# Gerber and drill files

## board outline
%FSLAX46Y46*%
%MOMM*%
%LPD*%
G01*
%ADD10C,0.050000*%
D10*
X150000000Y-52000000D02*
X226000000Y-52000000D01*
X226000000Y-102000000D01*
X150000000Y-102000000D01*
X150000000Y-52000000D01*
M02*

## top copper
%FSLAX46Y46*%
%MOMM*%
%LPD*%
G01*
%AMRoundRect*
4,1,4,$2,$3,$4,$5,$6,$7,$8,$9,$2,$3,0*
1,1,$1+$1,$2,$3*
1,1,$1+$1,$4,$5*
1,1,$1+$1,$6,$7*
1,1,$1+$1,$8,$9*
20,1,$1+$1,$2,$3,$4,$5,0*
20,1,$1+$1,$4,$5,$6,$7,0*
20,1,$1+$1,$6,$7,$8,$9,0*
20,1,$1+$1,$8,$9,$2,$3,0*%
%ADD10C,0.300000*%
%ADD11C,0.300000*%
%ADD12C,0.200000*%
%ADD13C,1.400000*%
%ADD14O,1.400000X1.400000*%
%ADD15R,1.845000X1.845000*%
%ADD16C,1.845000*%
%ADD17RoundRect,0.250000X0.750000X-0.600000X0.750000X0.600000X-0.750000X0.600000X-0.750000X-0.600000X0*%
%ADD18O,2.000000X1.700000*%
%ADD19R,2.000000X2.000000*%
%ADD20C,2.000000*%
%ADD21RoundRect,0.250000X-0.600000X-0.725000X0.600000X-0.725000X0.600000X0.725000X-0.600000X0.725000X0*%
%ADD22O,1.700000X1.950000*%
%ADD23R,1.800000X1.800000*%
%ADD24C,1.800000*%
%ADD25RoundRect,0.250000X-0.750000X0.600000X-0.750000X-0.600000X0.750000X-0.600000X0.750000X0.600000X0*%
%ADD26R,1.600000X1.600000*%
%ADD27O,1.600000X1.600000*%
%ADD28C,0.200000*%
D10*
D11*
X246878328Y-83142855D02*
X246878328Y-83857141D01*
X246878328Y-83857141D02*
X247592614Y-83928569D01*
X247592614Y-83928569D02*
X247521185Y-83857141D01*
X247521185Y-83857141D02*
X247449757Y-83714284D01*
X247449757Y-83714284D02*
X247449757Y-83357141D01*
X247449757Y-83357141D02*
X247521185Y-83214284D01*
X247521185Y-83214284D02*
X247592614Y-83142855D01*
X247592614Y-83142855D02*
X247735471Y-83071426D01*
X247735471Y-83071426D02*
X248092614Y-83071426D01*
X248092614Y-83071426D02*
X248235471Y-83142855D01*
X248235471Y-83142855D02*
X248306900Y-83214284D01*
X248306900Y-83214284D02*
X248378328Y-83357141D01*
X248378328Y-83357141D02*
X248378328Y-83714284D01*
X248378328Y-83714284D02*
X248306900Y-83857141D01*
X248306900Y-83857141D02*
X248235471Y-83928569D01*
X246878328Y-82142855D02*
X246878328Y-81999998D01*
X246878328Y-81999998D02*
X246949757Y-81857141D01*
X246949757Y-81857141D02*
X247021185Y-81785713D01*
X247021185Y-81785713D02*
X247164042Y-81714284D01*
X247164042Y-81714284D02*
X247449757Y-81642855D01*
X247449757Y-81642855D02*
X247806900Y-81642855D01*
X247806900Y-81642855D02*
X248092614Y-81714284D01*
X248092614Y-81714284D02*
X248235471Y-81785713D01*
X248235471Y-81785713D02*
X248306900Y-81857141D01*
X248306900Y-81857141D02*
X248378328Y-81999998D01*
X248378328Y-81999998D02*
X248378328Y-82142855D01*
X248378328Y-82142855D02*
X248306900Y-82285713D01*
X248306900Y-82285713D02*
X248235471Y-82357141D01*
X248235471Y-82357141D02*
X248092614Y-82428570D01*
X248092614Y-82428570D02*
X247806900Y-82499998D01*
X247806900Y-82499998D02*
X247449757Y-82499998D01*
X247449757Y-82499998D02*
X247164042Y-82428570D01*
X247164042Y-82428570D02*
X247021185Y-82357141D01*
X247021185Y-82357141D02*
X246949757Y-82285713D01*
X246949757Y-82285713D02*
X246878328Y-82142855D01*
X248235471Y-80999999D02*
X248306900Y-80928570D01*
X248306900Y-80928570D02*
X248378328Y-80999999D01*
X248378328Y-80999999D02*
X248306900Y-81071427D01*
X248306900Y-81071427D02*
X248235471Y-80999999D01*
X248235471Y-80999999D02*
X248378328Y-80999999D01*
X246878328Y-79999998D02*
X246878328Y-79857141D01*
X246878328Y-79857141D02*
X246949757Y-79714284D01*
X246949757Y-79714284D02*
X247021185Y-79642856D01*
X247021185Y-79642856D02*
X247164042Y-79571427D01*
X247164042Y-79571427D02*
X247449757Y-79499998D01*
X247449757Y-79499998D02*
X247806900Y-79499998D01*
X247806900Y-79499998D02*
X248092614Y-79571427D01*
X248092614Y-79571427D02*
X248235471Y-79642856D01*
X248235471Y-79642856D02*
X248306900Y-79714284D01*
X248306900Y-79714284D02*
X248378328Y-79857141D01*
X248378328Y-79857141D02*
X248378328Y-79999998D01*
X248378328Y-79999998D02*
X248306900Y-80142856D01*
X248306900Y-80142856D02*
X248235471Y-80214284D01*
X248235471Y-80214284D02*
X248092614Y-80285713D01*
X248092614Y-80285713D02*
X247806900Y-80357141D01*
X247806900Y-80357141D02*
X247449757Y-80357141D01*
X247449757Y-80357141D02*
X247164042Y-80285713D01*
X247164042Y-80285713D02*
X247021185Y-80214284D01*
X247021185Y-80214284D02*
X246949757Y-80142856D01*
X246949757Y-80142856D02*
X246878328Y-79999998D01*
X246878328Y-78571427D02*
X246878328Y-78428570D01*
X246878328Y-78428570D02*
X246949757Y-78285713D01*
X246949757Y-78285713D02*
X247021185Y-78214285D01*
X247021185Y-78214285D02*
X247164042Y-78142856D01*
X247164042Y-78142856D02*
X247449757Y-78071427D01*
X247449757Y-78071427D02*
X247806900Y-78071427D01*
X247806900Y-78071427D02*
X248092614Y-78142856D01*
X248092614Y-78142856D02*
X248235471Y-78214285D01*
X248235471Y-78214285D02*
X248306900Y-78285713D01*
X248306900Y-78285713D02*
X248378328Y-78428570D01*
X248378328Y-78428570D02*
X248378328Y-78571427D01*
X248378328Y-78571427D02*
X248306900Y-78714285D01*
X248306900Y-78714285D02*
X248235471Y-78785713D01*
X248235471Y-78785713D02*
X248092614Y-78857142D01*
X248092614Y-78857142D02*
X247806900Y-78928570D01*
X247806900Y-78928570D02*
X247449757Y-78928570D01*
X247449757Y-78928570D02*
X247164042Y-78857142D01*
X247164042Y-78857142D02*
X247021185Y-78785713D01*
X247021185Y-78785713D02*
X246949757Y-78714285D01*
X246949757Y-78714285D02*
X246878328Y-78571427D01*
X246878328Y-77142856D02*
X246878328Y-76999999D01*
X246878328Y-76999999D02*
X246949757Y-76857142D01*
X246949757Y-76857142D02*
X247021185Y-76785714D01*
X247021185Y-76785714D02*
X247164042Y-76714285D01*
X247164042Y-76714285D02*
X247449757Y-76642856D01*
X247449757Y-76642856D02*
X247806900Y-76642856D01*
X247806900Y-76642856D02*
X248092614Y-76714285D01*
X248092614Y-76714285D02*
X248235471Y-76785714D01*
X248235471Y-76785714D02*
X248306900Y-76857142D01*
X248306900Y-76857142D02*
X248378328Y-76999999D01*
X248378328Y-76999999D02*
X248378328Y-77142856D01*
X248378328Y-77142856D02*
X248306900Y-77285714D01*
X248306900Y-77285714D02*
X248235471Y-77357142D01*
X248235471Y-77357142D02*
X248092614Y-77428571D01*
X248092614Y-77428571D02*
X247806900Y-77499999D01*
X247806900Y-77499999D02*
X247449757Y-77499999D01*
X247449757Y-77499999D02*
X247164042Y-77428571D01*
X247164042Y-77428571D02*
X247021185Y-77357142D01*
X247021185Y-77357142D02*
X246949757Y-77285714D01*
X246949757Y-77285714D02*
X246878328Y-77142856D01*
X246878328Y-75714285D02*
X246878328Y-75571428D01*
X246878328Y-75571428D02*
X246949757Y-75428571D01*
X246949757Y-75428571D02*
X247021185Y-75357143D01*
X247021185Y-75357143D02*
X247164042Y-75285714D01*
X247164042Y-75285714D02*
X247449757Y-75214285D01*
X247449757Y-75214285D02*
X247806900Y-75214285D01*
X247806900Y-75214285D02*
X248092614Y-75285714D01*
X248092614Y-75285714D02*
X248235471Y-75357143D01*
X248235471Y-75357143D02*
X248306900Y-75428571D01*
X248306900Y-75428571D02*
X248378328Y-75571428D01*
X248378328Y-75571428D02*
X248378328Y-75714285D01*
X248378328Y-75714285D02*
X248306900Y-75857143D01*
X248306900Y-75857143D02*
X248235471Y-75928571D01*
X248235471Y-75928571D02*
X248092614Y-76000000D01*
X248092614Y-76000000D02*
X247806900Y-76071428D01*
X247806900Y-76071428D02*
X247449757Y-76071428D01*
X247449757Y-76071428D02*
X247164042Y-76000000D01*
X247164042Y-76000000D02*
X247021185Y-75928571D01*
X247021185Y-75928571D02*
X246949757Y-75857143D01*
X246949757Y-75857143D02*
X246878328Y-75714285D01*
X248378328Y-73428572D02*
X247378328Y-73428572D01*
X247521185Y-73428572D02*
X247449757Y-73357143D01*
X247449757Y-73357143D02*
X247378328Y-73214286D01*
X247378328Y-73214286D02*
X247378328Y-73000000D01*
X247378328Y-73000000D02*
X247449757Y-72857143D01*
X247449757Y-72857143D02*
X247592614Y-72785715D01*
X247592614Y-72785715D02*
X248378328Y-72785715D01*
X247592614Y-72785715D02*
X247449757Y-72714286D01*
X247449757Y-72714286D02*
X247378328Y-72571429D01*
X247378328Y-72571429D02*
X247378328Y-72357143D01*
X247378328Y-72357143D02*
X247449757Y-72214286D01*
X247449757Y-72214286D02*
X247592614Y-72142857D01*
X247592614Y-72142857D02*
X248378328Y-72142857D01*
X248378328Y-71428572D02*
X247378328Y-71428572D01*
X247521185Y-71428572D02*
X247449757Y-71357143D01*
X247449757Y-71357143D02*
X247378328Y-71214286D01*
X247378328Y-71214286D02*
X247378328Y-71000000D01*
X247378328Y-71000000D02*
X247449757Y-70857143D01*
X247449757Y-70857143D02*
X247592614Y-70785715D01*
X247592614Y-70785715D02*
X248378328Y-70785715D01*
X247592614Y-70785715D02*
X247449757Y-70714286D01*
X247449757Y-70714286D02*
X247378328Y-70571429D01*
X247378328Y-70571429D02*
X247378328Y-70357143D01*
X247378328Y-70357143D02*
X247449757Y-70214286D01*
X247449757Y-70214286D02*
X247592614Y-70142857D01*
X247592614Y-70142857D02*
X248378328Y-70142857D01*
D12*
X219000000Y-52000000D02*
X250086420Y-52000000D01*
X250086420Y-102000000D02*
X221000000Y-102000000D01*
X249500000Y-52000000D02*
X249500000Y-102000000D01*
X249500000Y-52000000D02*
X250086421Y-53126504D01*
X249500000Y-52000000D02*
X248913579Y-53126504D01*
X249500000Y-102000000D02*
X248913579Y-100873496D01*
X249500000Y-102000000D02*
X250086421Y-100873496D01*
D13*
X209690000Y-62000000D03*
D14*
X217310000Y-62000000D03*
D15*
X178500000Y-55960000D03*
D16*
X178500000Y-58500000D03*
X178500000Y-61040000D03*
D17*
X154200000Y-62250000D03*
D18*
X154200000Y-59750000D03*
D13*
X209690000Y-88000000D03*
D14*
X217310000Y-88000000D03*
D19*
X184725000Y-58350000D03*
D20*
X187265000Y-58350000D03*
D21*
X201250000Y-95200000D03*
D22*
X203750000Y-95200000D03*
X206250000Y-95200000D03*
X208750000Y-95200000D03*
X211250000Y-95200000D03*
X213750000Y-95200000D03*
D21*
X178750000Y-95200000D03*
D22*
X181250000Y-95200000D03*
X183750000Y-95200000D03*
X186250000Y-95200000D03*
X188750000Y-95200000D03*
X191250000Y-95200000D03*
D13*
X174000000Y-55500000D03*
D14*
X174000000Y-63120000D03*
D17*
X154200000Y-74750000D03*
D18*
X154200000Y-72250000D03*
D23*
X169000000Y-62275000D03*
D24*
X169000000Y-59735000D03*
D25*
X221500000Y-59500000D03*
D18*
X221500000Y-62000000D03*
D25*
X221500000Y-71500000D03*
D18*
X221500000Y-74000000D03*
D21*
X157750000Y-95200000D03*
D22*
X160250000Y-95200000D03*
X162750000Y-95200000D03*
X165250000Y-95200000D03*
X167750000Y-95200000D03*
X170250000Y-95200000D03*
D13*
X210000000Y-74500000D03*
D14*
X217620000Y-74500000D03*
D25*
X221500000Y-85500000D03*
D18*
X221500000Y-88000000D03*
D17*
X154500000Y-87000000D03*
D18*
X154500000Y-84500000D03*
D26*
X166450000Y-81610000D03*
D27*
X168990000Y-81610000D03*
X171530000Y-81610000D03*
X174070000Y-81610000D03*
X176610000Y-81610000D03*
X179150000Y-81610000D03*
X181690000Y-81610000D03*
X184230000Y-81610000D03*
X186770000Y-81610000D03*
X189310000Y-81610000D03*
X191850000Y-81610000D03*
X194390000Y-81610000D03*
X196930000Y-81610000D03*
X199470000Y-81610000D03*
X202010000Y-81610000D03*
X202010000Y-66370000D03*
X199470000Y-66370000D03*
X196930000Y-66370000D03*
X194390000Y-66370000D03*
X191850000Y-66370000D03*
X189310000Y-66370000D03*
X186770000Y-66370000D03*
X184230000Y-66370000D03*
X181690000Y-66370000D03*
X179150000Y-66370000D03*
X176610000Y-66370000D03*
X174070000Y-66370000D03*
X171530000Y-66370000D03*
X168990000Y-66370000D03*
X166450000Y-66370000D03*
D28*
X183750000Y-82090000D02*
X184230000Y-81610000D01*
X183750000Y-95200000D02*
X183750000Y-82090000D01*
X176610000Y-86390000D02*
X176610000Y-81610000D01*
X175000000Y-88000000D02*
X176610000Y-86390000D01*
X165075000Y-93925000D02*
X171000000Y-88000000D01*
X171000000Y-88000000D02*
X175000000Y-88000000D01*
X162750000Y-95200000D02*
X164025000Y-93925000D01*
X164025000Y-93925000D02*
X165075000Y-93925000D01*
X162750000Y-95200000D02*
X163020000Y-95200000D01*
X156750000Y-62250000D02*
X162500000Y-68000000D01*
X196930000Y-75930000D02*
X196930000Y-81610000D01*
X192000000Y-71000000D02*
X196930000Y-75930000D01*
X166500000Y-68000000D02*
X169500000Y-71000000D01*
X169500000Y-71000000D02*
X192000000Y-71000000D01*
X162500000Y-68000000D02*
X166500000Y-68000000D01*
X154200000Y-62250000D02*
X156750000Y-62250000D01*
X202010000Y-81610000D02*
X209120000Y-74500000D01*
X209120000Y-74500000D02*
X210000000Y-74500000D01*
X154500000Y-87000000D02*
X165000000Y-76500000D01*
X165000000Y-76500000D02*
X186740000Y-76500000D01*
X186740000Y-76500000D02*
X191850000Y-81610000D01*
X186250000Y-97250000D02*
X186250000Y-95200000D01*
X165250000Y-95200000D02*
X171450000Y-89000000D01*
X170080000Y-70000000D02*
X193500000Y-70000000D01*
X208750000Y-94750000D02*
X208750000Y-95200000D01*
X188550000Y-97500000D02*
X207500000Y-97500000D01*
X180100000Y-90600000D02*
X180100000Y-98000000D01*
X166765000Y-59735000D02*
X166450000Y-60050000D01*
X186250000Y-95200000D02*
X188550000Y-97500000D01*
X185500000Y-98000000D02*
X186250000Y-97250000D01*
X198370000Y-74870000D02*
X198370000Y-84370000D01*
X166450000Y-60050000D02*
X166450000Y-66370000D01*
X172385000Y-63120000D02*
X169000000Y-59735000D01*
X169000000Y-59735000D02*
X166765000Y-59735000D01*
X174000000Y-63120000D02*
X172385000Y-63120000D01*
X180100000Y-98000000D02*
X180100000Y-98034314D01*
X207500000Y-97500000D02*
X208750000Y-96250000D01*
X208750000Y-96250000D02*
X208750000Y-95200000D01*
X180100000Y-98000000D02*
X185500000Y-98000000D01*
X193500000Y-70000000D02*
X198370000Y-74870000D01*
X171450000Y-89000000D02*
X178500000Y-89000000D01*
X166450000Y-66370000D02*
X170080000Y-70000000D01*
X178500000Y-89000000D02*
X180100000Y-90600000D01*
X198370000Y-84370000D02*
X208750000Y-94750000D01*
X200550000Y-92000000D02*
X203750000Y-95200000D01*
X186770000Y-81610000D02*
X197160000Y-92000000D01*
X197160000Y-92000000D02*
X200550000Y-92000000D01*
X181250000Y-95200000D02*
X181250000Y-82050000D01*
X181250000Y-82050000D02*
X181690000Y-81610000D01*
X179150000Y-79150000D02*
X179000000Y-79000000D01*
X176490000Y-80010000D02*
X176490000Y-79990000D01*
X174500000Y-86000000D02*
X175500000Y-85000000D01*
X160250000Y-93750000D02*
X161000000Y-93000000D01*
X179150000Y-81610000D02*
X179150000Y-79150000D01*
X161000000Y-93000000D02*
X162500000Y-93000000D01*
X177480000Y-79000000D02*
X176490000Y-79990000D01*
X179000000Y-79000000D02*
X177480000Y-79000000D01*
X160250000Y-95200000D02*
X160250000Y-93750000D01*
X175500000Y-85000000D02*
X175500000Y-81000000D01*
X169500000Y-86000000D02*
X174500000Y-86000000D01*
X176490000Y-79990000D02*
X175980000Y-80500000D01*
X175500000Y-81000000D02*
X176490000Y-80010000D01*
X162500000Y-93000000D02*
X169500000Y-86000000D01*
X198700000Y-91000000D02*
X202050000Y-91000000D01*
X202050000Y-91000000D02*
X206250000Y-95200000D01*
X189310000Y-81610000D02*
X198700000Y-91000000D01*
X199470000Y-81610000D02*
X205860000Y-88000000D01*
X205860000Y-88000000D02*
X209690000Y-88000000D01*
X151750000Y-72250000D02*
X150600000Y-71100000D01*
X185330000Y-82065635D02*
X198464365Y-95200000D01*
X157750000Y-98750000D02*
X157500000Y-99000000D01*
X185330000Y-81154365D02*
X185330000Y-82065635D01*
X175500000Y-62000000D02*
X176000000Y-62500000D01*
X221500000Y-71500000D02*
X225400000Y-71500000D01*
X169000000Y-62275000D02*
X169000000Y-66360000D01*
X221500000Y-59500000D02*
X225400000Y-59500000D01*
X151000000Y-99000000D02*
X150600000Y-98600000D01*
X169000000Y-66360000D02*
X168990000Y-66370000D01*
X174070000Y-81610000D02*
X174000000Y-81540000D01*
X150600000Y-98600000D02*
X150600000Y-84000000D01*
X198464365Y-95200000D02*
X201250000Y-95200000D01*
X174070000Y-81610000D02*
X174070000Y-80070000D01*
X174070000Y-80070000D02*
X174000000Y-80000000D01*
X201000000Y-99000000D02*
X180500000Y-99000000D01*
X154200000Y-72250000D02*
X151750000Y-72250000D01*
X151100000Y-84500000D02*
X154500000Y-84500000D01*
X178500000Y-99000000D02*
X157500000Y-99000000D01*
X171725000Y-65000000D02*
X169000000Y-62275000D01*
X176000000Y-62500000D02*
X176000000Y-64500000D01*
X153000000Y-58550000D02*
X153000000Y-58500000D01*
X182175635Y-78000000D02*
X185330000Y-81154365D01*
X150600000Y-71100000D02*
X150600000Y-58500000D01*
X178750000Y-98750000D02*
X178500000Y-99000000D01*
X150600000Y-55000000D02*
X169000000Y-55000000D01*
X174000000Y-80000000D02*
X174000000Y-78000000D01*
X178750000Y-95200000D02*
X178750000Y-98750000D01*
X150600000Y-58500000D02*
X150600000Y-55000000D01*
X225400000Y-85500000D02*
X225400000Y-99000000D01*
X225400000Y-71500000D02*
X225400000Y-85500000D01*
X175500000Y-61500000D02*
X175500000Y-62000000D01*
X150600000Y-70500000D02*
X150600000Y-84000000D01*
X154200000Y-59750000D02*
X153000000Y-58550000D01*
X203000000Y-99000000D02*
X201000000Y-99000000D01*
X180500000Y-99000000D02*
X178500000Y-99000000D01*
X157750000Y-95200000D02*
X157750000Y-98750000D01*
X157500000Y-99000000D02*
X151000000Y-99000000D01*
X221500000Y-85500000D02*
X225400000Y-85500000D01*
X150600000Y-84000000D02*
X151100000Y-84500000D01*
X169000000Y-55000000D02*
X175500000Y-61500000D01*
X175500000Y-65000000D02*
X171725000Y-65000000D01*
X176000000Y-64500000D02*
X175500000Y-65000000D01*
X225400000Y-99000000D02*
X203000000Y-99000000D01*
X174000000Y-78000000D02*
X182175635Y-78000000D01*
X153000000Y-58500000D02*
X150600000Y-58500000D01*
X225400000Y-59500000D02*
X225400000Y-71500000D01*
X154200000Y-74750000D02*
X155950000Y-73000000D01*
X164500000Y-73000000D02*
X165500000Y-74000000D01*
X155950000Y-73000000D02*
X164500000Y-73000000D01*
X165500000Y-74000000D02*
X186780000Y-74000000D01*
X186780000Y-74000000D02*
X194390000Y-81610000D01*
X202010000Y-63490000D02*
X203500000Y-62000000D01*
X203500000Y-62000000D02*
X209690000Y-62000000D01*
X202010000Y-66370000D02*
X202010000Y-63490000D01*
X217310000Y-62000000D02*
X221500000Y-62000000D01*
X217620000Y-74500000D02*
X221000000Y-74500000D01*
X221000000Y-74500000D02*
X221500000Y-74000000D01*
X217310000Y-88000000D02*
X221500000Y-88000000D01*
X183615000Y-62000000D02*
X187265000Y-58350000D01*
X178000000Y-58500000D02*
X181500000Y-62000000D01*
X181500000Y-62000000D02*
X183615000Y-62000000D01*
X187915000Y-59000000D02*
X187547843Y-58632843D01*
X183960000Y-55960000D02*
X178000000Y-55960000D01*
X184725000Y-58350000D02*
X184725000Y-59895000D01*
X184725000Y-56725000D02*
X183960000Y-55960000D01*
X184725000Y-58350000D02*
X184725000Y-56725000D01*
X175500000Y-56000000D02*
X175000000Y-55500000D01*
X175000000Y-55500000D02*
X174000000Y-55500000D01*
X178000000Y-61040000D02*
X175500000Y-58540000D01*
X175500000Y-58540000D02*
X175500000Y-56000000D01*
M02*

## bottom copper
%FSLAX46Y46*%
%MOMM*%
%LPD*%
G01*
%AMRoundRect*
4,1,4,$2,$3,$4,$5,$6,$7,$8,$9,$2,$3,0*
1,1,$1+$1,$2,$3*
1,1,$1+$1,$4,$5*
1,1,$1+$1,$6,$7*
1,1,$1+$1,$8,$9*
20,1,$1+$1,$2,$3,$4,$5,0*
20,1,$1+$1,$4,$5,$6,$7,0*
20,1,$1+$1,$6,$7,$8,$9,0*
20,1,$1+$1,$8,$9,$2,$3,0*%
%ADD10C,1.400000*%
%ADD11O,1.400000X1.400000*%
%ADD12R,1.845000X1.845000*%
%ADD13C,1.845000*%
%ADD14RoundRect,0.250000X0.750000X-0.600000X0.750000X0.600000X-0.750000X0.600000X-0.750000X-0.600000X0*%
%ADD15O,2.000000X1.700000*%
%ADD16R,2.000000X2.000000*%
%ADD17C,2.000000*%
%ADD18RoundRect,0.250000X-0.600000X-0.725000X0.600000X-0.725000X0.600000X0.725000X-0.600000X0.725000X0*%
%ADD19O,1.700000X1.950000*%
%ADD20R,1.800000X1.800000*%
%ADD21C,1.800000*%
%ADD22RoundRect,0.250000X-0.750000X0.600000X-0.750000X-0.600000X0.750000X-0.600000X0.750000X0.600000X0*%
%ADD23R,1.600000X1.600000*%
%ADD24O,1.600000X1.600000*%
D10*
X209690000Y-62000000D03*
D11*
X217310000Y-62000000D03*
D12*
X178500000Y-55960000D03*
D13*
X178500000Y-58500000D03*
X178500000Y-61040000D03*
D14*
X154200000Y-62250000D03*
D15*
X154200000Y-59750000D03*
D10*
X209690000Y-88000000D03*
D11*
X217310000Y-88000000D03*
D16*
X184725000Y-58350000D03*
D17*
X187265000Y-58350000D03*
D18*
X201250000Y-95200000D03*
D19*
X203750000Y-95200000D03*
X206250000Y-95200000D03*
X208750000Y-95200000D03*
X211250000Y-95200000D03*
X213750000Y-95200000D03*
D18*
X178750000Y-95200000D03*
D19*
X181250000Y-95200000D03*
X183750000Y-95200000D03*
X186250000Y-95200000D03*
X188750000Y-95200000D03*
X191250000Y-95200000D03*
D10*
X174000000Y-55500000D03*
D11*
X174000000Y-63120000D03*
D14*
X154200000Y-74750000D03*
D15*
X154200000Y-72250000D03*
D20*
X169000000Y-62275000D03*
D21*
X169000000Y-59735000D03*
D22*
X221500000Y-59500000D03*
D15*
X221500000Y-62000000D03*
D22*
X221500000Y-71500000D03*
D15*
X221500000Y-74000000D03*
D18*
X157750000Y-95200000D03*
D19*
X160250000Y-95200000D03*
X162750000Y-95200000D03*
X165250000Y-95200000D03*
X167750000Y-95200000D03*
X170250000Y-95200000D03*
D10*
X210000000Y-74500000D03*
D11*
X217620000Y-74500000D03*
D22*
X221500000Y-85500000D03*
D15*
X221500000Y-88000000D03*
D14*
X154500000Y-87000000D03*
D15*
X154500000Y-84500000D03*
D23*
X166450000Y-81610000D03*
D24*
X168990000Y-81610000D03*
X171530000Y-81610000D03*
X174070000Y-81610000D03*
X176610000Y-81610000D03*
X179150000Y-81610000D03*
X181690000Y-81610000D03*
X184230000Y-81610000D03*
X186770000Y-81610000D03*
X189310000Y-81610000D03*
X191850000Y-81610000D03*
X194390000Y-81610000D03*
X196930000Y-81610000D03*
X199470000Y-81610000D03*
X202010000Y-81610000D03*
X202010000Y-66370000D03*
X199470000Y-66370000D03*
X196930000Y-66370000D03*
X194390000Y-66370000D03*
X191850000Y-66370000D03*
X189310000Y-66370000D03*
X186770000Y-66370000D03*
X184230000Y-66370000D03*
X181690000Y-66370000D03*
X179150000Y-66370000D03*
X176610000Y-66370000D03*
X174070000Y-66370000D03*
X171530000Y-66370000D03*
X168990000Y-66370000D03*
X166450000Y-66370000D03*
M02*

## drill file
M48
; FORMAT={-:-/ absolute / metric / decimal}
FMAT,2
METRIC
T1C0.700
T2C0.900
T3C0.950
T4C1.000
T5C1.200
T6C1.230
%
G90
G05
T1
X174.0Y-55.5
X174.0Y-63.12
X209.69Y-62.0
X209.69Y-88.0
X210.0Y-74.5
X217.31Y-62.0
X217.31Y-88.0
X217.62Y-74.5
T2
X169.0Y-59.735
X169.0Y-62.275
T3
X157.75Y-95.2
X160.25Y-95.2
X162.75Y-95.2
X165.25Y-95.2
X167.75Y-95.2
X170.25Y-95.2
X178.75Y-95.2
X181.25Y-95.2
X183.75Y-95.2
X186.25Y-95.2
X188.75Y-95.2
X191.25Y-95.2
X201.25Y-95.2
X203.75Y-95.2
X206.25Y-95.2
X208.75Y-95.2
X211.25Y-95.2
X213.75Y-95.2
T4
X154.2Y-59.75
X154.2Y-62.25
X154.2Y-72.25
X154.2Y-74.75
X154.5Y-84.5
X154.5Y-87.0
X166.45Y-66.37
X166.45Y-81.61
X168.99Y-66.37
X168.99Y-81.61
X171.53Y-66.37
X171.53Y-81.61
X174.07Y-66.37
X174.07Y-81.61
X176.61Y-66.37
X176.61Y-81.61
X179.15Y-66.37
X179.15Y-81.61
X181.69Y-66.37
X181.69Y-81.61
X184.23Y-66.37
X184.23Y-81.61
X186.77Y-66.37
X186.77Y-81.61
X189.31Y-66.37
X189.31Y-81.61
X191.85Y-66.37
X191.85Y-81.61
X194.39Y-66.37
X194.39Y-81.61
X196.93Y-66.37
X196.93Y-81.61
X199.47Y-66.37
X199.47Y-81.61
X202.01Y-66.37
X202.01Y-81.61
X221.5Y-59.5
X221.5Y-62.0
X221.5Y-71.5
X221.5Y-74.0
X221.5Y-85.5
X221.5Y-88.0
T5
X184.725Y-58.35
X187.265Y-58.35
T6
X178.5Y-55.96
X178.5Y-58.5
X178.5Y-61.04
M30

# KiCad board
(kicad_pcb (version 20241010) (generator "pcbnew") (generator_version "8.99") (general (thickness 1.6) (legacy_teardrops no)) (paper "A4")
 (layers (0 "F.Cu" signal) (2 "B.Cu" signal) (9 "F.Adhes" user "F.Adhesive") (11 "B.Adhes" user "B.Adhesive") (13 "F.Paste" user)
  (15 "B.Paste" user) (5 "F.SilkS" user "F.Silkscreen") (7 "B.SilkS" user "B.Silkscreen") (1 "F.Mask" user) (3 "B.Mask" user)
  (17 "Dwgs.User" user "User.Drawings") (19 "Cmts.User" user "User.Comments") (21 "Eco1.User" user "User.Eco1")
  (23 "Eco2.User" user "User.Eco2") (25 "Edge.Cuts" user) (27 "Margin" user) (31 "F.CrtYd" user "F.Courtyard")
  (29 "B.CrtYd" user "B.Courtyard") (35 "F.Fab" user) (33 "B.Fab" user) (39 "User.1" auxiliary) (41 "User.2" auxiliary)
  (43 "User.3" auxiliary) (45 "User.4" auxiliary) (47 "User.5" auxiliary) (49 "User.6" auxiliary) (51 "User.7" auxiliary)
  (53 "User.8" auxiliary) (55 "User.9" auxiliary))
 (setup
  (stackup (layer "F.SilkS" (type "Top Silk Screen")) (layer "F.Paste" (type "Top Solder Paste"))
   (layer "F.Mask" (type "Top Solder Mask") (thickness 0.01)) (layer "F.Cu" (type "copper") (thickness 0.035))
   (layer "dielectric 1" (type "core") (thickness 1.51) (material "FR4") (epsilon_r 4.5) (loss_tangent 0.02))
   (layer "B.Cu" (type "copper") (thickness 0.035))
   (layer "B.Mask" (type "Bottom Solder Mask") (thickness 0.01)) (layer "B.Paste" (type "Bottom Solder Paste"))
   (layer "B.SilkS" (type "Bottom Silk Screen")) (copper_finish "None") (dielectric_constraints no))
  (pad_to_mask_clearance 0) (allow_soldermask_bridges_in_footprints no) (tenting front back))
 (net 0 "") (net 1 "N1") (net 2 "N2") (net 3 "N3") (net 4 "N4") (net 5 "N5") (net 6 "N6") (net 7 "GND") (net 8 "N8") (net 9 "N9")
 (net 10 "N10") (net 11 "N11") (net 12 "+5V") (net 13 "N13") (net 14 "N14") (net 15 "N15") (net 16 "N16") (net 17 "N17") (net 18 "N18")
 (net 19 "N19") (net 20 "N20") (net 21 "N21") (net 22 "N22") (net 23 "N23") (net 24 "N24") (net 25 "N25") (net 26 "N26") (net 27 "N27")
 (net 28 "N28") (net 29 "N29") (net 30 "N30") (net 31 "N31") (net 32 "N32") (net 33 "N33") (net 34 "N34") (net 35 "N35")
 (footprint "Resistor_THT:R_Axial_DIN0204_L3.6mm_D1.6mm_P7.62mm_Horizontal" (layer "F.Cu") (at 209.69 62)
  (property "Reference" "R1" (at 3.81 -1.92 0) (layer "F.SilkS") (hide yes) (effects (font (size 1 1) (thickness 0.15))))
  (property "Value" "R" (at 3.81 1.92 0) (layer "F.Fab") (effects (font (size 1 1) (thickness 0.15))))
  (pad "1" thru_hole circle (at 0 0) (size 1.4 1.4) (drill 0.7) (layers "*.Cu" "*.Mask") (remove_unused_layers no) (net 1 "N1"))
  (pad "2" thru_hole oval (at 7.62 0) (size 1.4 1.4) (drill 0.7) (layers "*.Cu" "*.Mask") (remove_unused_layers no) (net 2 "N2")))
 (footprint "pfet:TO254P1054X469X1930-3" (layer "F.Cu") (at 179.3105 58.5 -90)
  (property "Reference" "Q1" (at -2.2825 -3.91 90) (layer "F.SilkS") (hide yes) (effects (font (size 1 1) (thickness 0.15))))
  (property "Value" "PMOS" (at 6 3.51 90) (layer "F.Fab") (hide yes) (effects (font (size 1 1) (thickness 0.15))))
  (pad "1" thru_hole rect (at -2.54 0.8105 270) (size 1.845 1.845) (drill 1.23) (layers "*.Cu" "*.Mask") (remove_unused_layers no)
   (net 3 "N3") (solder_mask_margin 0.102))
  (pad "2" thru_hole circle (at 0 0.8105 270) (size 1.845 1.845) (drill 1.23) (layers "*.Cu" "*.Mask") (remove_unused_layers no)
   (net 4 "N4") (solder_mask_margin 0.102))
  (pad "3" thru_hole circle (at 2.54 0.8105 270) (size 1.845 1.845) (drill 1.23) (layers "*.Cu" "*.Mask") (remove_unused_layers no)
   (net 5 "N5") (solder_mask_margin 0.102)))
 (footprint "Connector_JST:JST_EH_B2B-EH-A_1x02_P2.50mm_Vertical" (layer "F.Cu") (at 154.2 62.25 90)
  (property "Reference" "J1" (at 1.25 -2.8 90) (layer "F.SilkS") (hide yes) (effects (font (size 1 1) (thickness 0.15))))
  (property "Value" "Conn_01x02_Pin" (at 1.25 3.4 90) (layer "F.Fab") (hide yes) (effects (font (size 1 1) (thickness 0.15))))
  (pad "1" thru_hole roundrect (at 0 0 90) (size 1.7 2) (drill 1) (layers "*.Cu" "*.Mask") (remove_unused_layers no)
   (roundrect_rratio 0.147059) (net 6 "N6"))
  (pad "2" thru_hole oval (at 2.5 0 90) (size 1.7 2) (drill 1) (layers "*.Cu" "*.Mask") (remove_unused_layers no) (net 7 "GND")))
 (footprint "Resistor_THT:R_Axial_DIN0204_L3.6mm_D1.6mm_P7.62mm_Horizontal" (layer "F.Cu") (at 209.69 88)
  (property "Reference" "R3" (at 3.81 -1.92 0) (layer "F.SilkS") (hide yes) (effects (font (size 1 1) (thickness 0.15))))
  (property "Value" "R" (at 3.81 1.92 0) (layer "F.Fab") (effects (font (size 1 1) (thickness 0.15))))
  (pad "1" thru_hole circle (at 0 0) (size 1.4 1.4) (drill 0.7) (layers "*.Cu" "*.Mask") (remove_unused_layers no) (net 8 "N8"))
  (pad "2" thru_hole oval (at 7.62 0) (size 1.4 1.4) (drill 0.7) (layers "*.Cu" "*.Mask") (remove_unused_layers no) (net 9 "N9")))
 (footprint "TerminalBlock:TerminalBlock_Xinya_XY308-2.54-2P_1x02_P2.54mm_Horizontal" (layer "F.Cu") (at 184.725 58.35)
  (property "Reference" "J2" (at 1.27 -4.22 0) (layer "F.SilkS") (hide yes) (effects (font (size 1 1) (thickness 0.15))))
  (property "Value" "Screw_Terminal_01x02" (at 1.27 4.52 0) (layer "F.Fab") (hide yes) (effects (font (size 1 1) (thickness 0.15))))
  (pad "1" thru_hole rect (at 0 0) (size 2 2) (drill 1.2) (layers "*.Cu" "*.Mask") (remove_unused_layers no) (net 3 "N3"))
  (pad "2" thru_hole circle (at 2.54 0) (size 2 2) (drill 1.2) (layers "*.Cu" "*.Mask") (remove_unused_layers no) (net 4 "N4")))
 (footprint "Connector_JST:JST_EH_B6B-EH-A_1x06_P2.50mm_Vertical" (layer "F.Cu") (at 201.25 95.2)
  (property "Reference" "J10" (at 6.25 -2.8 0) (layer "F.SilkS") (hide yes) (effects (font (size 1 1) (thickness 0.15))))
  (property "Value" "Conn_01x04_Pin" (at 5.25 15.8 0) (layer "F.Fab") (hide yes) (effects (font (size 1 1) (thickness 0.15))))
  (pad "1" thru_hole roundrect (at 0 0) (size 1.7 1.95) (drill 0.95) (layers "*.Cu" "*.Mask") (remove_unused_layers no)
   (roundrect_rratio 0.147059) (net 7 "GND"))
  (pad "2" thru_hole oval (at 2.5 0) (size 1.7 1.95) (drill 0.95) (layers "*.Cu" "*.Mask") (remove_unused_layers no) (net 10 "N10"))
  (pad "3" thru_hole oval (at 5 0) (size 1.7 1.95) (drill 0.95) (layers "*.Cu" "*.Mask") (remove_unused_layers no) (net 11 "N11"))
  (pad "4" thru_hole oval (at 7.5 0) (size 1.7 1.95) (drill 0.95) (layers "*.Cu" "*.Mask") (remove_unused_layers no) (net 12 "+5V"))
  (pad "5" thru_hole oval (at 10 0) (size 1.7 1.95) (drill 0.95) (layers "*.Cu" "*.Mask") (remove_unused_layers no))
  (pad "6" thru_hole oval (at 12.5 0) (size 1.7 1.95) (drill 0.95) (layers "*.Cu" "*.Mask") (remove_unused_layers no)))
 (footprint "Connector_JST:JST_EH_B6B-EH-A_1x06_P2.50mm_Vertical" (layer "F.Cu") (at 178.75 95.2)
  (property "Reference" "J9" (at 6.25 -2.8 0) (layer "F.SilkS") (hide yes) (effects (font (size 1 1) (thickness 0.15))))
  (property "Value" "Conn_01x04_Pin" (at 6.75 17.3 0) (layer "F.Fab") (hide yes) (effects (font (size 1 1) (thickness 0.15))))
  (pad "1" thru_hole roundrect (at 0 0) (size 1.7 1.95) (drill 0.95) (layers "*.Cu" "*.Mask") (remove_unused_layers no)
   (roundrect_rratio 0.147059) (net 7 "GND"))
  (pad "2" thru_hole oval (at 2.5 0) (size 1.7 1.95) (drill 0.95) (layers "*.Cu" "*.Mask") (remove_unused_layers no) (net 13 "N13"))
  (pad "3" thru_hole oval (at 5 0) (size 1.7 1.95) (drill 0.95) (layers "*.Cu" "*.Mask") (remove_unused_layers no) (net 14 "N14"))
  (pad "4" thru_hole oval (at 7.5 0) (size 1.7 1.95) (drill 0.95) (layers "*.Cu" "*.Mask") (remove_unused_layers no) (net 12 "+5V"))
  (pad "5" thru_hole oval (at 10 0) (size 1.7 1.95) (drill 0.95) (layers "*.Cu" "*.Mask") (remove_unused_layers no))
  (pad "6" thru_hole oval (at 12.5 0) (size 1.7 1.95) (drill 0.95) (layers "*.Cu" "*.Mask") (remove_unused_layers no)))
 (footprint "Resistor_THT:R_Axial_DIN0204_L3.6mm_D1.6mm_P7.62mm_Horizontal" (layer "F.Cu") (at 174 55.5 -90)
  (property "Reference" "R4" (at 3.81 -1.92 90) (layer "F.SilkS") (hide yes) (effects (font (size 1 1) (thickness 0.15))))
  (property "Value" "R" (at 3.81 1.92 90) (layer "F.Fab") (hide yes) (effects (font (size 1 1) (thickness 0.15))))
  (pad "1" thru_hole circle (at 0 0 270) (size 1.4 1.4) (drill 0.7) (layers "*.Cu" "*.Mask") (remove_unused_layers no) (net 5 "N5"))
  (pad "2" thru_hole oval (at 7.62 0 270) (size 1.4 1.4) (drill 0.7) (layers "*.Cu" "*.Mask") (remove_unused_layers no) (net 12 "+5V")))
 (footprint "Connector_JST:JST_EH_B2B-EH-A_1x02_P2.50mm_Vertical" (layer "F.Cu") (at 154.2 74.75 90)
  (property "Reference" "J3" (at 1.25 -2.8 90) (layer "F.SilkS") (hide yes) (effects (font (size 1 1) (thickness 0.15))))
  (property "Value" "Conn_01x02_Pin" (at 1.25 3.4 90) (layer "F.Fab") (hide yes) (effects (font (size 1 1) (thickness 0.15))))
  (pad "1" thru_hole roundrect (at 0 0 90) (size 1.7 2) (drill 1) (layers "*.Cu" "*.Mask") (remove_unused_layers no)
   (roundrect_rratio 0.147059) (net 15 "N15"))
  (pad "2" thru_hole oval (at 2.5 0 90) (size 1.7 2) (drill 1) (layers "*.Cu" "*.Mask") (remove_unused_layers no) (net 7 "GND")))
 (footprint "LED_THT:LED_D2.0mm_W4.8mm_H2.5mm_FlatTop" (layer "F.Cu") (at 169 62.275 90)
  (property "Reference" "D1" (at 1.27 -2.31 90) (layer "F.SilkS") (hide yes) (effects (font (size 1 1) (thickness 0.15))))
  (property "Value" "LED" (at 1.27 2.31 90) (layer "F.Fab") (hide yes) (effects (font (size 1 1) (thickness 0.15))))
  (pad "1" thru_hole rect (at 0 0 90) (size 1.8 1.8) (drill 0.9) (layers "*.Cu" "*.Mask") (remove_unused_layers no) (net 7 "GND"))
  (pad "2" thru_hole circle (at 2.54 0 90) (size 1.8 1.8) (drill 0.9) (layers "*.Cu" "*.Mask") (remove_unused_layers no) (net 12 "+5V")))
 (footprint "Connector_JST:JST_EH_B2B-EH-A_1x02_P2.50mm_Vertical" (layer "F.Cu") (at 221.5 59.5 -90)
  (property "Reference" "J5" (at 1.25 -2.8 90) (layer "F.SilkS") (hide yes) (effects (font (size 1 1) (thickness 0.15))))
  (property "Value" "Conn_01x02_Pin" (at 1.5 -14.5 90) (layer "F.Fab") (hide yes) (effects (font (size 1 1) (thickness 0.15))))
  (pad "1" thru_hole roundrect (at 0 0 270) (size 1.7 2) (drill 1) (layers "*.Cu" "*.Mask") (remove_unused_layers no)
   (roundrect_rratio 0.147059) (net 7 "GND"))
  (pad "2" thru_hole oval (at 2.5 0 270) (size 1.7 2) (drill 1) (layers "*.Cu" "*.Mask") (remove_unused_layers no) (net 2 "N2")))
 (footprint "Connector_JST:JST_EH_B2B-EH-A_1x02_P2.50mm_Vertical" (layer "F.Cu") (at 221.5 71.5 -90)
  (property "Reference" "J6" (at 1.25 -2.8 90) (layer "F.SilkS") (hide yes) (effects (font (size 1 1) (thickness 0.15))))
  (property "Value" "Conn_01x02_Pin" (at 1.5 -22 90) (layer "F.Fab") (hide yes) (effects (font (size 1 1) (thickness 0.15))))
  (pad "1" thru_hole roundrect (at 0 0 270) (size 1.7 2) (drill 1) (layers "*.Cu" "*.Mask") (remove_unused_layers no)
   (roundrect_rratio 0.147059) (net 7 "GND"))
  (pad "2" thru_hole oval (at 2.5 0 270) (size 1.7 2) (drill 1) (layers "*.Cu" "*.Mask") (remove_unused_layers no) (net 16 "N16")))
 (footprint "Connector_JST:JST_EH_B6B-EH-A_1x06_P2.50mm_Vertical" (layer "F.Cu") (at 157.75 95.2)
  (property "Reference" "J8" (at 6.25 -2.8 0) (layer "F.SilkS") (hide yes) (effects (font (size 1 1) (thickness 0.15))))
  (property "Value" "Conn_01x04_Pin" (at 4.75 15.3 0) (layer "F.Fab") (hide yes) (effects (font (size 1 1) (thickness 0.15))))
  (pad "1" thru_hole roundrect (at 0 0) (size 1.7 1.95) (drill 0.95) (layers "*.Cu" "*.Mask") (remove_unused_layers no)
   (roundrect_rratio 0.147059) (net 7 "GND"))
  (pad "2" thru_hole oval (at 2.5 0) (size 1.7 1.95) (drill 0.95) (layers "*.Cu" "*.Mask") (remove_unused_layers no) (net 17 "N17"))
  (pad "3" thru_hole oval (at 5 0) (size 1.7 1.95) (drill 0.95) (layers "*.Cu" "*.Mask") (remove_unused_layers no) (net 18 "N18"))
  (pad "4" thru_hole oval (at 7.5 0) (size 1.7 1.95) (drill 0.95) (layers "*.Cu" "*.Mask") (remove_unused_layers no) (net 12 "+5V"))
  (pad "5" thru_hole oval (at 10 0) (size 1.7 1.95) (drill 0.95) (layers "*.Cu" "*.Mask") (remove_unused_layers no))
  (pad "6" thru_hole oval (at 12.5 0) (size 1.7 1.95) (drill 0.95) (layers "*.Cu" "*.Mask") (remove_unused_layers no)))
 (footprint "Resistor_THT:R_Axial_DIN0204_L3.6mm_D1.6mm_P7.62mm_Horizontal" (layer "F.Cu") (at 210 74.5)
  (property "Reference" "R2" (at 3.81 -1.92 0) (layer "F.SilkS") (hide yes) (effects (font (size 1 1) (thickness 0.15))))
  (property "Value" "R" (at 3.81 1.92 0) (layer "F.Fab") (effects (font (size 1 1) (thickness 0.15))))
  (pad "1" thru_hole circle (at 0 0) (size 1.4 1.4) (drill 0.7) (layers "*.Cu" "*.Mask") (remove_unused_layers no) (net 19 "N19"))
  (pad "2" thru_hole oval (at 7.62 0) (size 1.4 1.4) (drill 0.7) (layers "*.Cu" "*.Mask") (remove_unused_layers no) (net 16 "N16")))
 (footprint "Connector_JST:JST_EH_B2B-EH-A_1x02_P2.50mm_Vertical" (layer "F.Cu") (at 221.5 85.5 -90)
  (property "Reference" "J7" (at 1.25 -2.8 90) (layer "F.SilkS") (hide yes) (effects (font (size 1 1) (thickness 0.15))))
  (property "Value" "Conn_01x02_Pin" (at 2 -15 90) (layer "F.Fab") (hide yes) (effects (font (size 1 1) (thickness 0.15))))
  (pad "1" thru_hole roundrect (at 0 0 270) (size 1.7 2) (drill 1) (layers "*.Cu" "*.Mask") (remove_unused_layers no)
   (roundrect_rratio 0.147059) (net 7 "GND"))
  (pad "2" thru_hole oval (at 2.5 0 270) (size 1.7 2) (drill 1) (layers "*.Cu" "*.Mask") (remove_unused_layers no) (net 9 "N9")))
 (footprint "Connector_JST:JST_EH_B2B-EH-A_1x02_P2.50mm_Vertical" (layer "F.Cu") (at 154.5 87 90)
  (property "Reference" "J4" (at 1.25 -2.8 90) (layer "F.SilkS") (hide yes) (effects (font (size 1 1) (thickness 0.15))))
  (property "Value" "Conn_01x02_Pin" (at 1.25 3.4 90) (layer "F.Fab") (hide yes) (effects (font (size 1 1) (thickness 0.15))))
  (pad "1" thru_hole roundrect (at 0 0 90) (size 1.7 2) (drill 1) (layers "*.Cu" "*.Mask") (remove_unused_layers no)
   (roundrect_rratio 0.147059) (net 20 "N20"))
  (pad "2" thru_hole oval (at 2.5 0 90) (size 1.7 2) (drill 1) (layers "*.Cu" "*.Mask") (remove_unused_layers no) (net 7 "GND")))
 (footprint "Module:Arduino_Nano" (layer "F.Cu") (at 166.45 81.61 90)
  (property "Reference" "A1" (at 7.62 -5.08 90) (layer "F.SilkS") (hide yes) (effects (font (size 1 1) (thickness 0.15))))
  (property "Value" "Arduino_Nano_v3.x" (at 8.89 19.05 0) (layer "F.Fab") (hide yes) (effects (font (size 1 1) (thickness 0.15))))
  (pad "1" thru_hole rect (at 0 0 90) (size 1.6 1.6) (drill 1) (layers "*.Cu" "*.Mask") (remove_unused_layers no) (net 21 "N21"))
  (pad "2" thru_hole oval (at 0 2.54 90) (size 1.6 1.6) (drill 1) (layers "*.Cu" "*.Mask") (remove_unused_layers no) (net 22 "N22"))
  (pad "3" thru_hole oval (at 0 5.08 90) (size 1.6 1.6) (drill 1) (layers "*.Cu" "*.Mask") (remove_unused_layers no) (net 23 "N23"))
  (pad "4" thru_hole oval (at 0 7.62 90) (size 1.6 1.6) (drill 1) (layers "*.Cu" "*.Mask") (remove_unused_layers no) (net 7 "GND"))
  (pad "5" thru_hole oval (at 0 10.16 90) (size 1.6 1.6) (drill 1) (layers "*.Cu" "*.Mask") (remove_unused_layers no) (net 18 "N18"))
  (pad "6" thru_hole oval (at 0 12.7 90) (size 1.6 1.6) (drill 1) (layers "*.Cu" "*.Mask") (remove_unused_layers no) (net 17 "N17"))
  (pad "7" thru_hole oval (at 0 15.24 90) (size 1.6 1.6) (drill 1) (layers "*.Cu" "*.Mask") (remove_unused_layers no) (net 13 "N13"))
  (pad "8" thru_hole oval (at 0 17.78 90) (size 1.6 1.6) (drill 1) (layers "*.Cu" "*.Mask") (remove_unused_layers no) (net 14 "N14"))
  (pad "9" thru_hole oval (at 0 20.32 90) (size 1.6 1.6) (drill 1) (layers "*.Cu" "*.Mask") (remove_unused_layers no) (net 10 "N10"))
  (pad "10" thru_hole oval (at 0 22.86 90) (size 1.6 1.6) (drill 1) (layers "*.Cu" "*.Mask") (remove_unused_layers no) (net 11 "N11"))
  (pad "11" thru_hole oval (at 0 25.4 90) (size 1.6 1.6) (drill 1) (layers "*.Cu" "*.Mask") (remove_unused_layers no) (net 20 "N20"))
  (pad "12" thru_hole oval (at 0 27.94 90) (size 1.6 1.6) (drill 1) (layers "*.Cu" "*.Mask") (remove_unused_layers no) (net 15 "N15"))
  (pad "13" thru_hole oval (at 0 30.48 90) (size 1.6 1.6) (drill 1) (layers "*.Cu" "*.Mask") (remove_unused_layers no) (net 6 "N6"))
  (pad "14" thru_hole oval (at 0 33.02 90) (size 1.6 1.6) (drill 1) (layers "*.Cu" "*.Mask") (remove_unused_layers no) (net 8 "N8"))
  (pad "15" thru_hole oval (at 0 35.56 90) (size 1.6 1.6) (drill 1) (layers "*.Cu" "*.Mask") (remove_unused_layers no) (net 19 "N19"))
  (pad "16" thru_hole oval (at 15.24 35.56 90) (size 1.6 1.6) (drill 1) (layers "*.Cu" "*.Mask") (remove_unused_layers no) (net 1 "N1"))
  (pad "17" thru_hole oval (at 15.24 33.02 90) (size 1.6 1.6) (drill 1) (layers "*.Cu" "*.Mask") (remove_unused_layers no) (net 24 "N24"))
  (pad "18" thru_hole oval (at 15.24 30.48 90) (size 1.6 1.6) (drill 1) (layers "*.Cu" "*.Mask") (remove_unused_layers no) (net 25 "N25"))
  (pad "19" thru_hole oval (at 15.24 27.94 90) (size 1.6 1.6) (drill 1) (layers "*.Cu" "*.Mask") (remove_unused_layers no) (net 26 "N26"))
  (pad "20" thru_hole oval (at 15.24 25.4 90) (size 1.6 1.6) (drill 1) (layers "*.Cu" "*.Mask") (remove_unused_layers no) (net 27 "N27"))
  (pad "21" thru_hole oval (at 15.24 22.86 90) (size 1.6 1.6) (drill 1) (layers "*.Cu" "*.Mask") (remove_unused_layers no) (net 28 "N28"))
  (pad "22" thru_hole oval (at 15.24 20.32 90) (size 1.6 1.6) (drill 1) (layers "*.Cu" "*.Mask") (remove_unused_layers no) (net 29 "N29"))
  (pad "23" thru_hole oval (at 15.24 17.78 90) (size 1.6 1.6) (drill 1) (layers "*.Cu" "*.Mask") (remove_unused_layers no) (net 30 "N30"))
  (pad "24" thru_hole oval (at 15.24 15.24 90) (size 1.6 1.6) (drill 1) (layers "*.Cu" "*.Mask") (remove_unused_layers no) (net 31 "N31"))
  (pad "25" thru_hole oval (at 15.24 12.7 90) (size 1.6 1.6) (drill 1) (layers "*.Cu" "*.Mask") (remove_unused_layers no) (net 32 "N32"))
  (pad "26" thru_hole oval (at 15.24 10.16 90) (size 1.6 1.6) (drill 1) (layers "*.Cu" "*.Mask") (remove_unused_layers no) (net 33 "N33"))
  (pad "27" thru_hole oval (at 15.24 7.62 90) (size 1.6 1.6) (drill 1) (layers "*.Cu" "*.Mask") (remove_unused_layers no) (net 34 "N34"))
  (pad "28" thru_hole oval (at 15.24 5.08 90) (size 1.6 1.6) (drill 1) (layers "*.Cu" "*.Mask") (remove_unused_layers no) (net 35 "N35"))
  (pad "29" thru_hole oval (at 15.24 2.54 90) (size 1.6 1.6) (drill 1) (layers "*.Cu" "*.Mask") (remove_unused_layers no) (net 7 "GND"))
  (pad "30" thru_hole oval (at 15.24 0 90) (size 1.6 1.6) (drill 1) (layers "*.Cu" "*.Mask") (remove_unused_layers no) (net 12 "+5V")))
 (gr_rect (start 150 52) (end 226 102) (stroke (width 0.05) (type default)) (fill none) (layer "Edge.Cuts"))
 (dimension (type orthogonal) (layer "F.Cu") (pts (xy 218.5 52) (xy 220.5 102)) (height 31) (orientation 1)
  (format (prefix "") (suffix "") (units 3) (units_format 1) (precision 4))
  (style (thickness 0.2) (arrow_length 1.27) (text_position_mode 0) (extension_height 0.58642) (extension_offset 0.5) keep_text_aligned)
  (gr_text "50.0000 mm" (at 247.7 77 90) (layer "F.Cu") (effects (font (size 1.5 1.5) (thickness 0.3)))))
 (segment (start 183.75 82.09) (end 184.23 81.61) (width 0.2) (layer "F.Cu") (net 14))
 (segment (start 183.75 95.2) (end 183.75 82.09) (width 0.2) (layer "F.Cu") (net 14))
 (segment (start 176.61 86.39) (end 176.61 81.61) (width 0.2) (layer "F.Cu") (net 18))
 (segment (start 175 88) (end 176.61 86.39) (width 0.2) (layer "F.Cu") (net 18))
 (segment (start 165.075 93.925) (end 171 88) (width 0.2) (layer "F.Cu") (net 18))
 (segment (start 171 88) (end 175 88) (width 0.2) (layer "F.Cu") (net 18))
 (segment (start 162.75 95.2) (end 164.025 93.925) (width 0.2) (layer "F.Cu") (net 18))
 (segment (start 164.025 93.925) (end 165.075 93.925) (width 0.2) (layer "F.Cu") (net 18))
 (segment (start 162.75 95.2) (end 163.02 95.2) (width 0.2) (layer "F.Cu") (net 18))
 (segment (start 156.75 62.25) (end 162.5 68) (width 0.2) (layer "F.Cu") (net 6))
 (segment (start 196.93 75.93) (end 196.93 81.61) (width 0.2) (layer "F.Cu") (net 6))
 (segment (start 192 71) (end 196.93 75.93) (width 0.2) (layer "F.Cu") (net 6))
 (segment (start 166.5 68) (end 169.5 71) (width 0.2) (layer "F.Cu") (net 6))
 (segment (start 169.5 71) (end 192 71) (width 0.2) (layer "F.Cu") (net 6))
 (segment (start 162.5 68) (end 166.5 68) (width 0.2) (layer "F.Cu") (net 6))
 (segment (start 154.2 62.25) (end 156.75 62.25) (width 0.2) (layer "F.Cu") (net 6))
 (segment (start 202.01 81.61) (end 209.12 74.5) (width 0.2) (layer "F.Cu") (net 19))
 (segment (start 209.12 74.5) (end 210 74.5) (width 0.2) (layer "F.Cu") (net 19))
 (segment (start 154.5 87) (end 165 76.5) (width 0.2) (layer "F.Cu") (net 20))
 (segment (start 165 76.5) (end 186.74 76.5) (width 0.2) (layer "F.Cu") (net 20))
 (segment (start 186.74 76.5) (end 191.85 81.61) (width 0.2) (layer "F.Cu") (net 20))
 (segment (start 186.25 97.25) (end 186.25 95.2) (width 0.2) (layer "F.Cu") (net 12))
 (segment (start 165.25 95.2) (end 171.45 89) (width 0.2) (layer "F.Cu") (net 12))
 (segment (start 170.08 70) (end 193.5 70) (width 0.2) (layer "F.Cu") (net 12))
 (segment (start 208.75 94.75) (end 208.75 95.2) (width 0.2) (layer "F.Cu") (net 12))
 (segment (start 188.55 97.5) (end 207.5 97.5) (width 0.2) (layer "F.Cu") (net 12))
 (segment (start 180.1 90.6) (end 180.1 98) (width 0.2) (layer "F.Cu") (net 12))
 (segment (start 166.765 59.735) (end 166.45 60.05) (width 0.2) (layer "F.Cu") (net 12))
 (segment (start 186.25 95.2) (end 188.55 97.5) (width 0.2) (layer "F.Cu") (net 12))
 (segment (start 185.5 98) (end 186.25 97.25) (width 0.2) (layer "F.Cu") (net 12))
 (segment (start 198.37 74.87) (end 198.37 84.37) (width 0.2) (layer "F.Cu") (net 12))
 (segment (start 166.45 60.05) (end 166.45 66.37) (width 0.2) (layer "F.Cu") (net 12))
 (segment (start 172.385 63.12) (end 169 59.735) (width 0.2) (layer "F.Cu") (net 12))
 (segment (start 169 59.735) (end 166.765 59.735) (width 0.2) (layer "F.Cu") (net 12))
 (segment (start 174 63.12) (end 172.385 63.12) (width 0.2) (layer "F.Cu") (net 12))
 (segment (start 180.1 98) (end 180.1 98.034314) (width 0.2) (layer "F.Cu") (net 12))
 (segment (start 207.5 97.5) (end 208.75 96.25) (width 0.2) (layer "F.Cu") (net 12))
 (segment (start 208.75 96.25) (end 208.75 95.2) (width 0.2) (layer "F.Cu") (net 12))
 (segment (start 180.1 98) (end 185.5 98) (width 0.2) (layer "F.Cu") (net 12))
 (segment (start 193.5 70) (end 198.37 74.87) (width 0.2) (layer "F.Cu") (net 12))
 (segment (start 171.45 89) (end 178.5 89) (width 0.2) (layer "F.Cu") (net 12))
 (segment (start 166.45 66.37) (end 170.08 70) (width 0.2) (layer "F.Cu") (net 12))
 (segment (start 178.5 89) (end 180.1 90.6) (width 0.2) (layer "F.Cu") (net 12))
 (segment (start 198.37 84.37) (end 208.75 94.75) (width 0.2) (layer "F.Cu") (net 12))
 (segment (start 200.55 92) (end 203.75 95.2) (width 0.2) (layer "F.Cu") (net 10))
 (segment (start 186.77 81.61) (end 197.16 92) (width 0.2) (layer "F.Cu") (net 10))
 (segment (start 197.16 92) (end 200.55 92) (width 0.2) (layer "F.Cu") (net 10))
 (segment (start 181.25 95.2) (end 181.25 82.05) (width 0.2) (layer "F.Cu") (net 13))
 (segment (start 181.25 82.05) (end 181.69 81.61) (width 0.2) (layer "F.Cu") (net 13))
 (segment (start 179.15 79.15) (end 179 79) (width 0.2) (layer "F.Cu") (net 17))
 (segment (start 176.49 80.01) (end 176.49 79.99) (width 0.2) (layer "F.Cu") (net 17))
 (segment (start 174.5 86) (end 175.5 85) (width 0.2) (layer "F.Cu") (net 17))
 (segment (start 160.25 93.75) (end 161 93) (width 0.2) (layer "F.Cu") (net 17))
 (segment (start 179.15 81.61) (end 179.15 79.15) (width 0.2) (layer "F.Cu") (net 17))
 (segment (start 161 93) (end 162.5 93) (width 0.2) (layer "F.Cu") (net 17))
 (segment (start 177.48 79) (end 176.49 79.99) (width 0.2) (layer "F.Cu") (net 17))
 (segment (start 179 79) (end 177.48 79) (width 0.2) (layer "F.Cu") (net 17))
 (segment (start 160.25 95.2) (end 160.25 93.75) (width 0.2) (layer "F.Cu") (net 17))
 (segment (start 175.5 85) (end 175.5 81) (width 0.2) (layer "F.Cu") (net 17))
 (segment (start 169.5 86) (end 174.5 86) (width 0.2) (layer "F.Cu") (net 17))
 (segment (start 176.49 79.99) (end 175.98 80.5) (width 0.2) (layer "F.Cu") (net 17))
 (segment (start 175.5 81) (end 176.49 80.01) (width 0.2) (layer "F.Cu") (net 17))
 (segment (start 162.5 93) (end 169.5 86) (width 0.2) (layer "F.Cu") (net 17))
 (segment (start 198.7 91) (end 202.05 91) (width 0.2) (layer "F.Cu") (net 11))
 (segment (start 202.05 91) (end 206.25 95.2) (width 0.2) (layer "F.Cu") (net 11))
 (segment (start 189.31 81.61) (end 198.7 91) (width 0.2) (layer "F.Cu") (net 11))
 (segment (start 199.47 81.61) (end 205.86 88) (width 0.2) (layer "F.Cu") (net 8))
 (segment (start 205.86 88) (end 209.69 88) (width 0.2) (layer "F.Cu") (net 8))
 (segment (start 151.75 72.25) (end 150.6 71.1) (width 0.2) (layer "F.Cu") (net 7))
 (segment (start 185.33 82.065635) (end 198.464365 95.2) (width 0.2) (layer "F.Cu") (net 7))
 (segment (start 157.75 98.75) (end 157.5 99) (width 0.2) (layer "F.Cu") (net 7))
 (segment (start 185.33 81.154365) (end 185.33 82.065635) (width 0.2) (layer "F.Cu") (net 7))
 (segment (start 175.5 62) (end 176 62.5) (width 0.2) (layer "F.Cu") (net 7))
 (segment (start 221.5 71.5) (end 225.4 71.5) (width 0.2) (layer "F.Cu") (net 7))
 (segment (start 169 62.275) (end 169 66.36) (width 0.2) (layer "F.Cu") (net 7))
 (segment (start 221.5 59.5) (end 225.4 59.5) (width 0.2) (layer "F.Cu") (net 7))
 (segment (start 151 99) (end 150.6 98.6) (width 0.2) (layer "F.Cu") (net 7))
 (segment (start 169 66.36) (end 168.99 66.37) (width 0.2) (layer "F.Cu") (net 7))
 (segment (start 174.07 81.61) (end 174 81.54) (width 0.2) (layer "F.Cu") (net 7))
 (segment (start 150.6 98.6) (end 150.6 84) (width 0.2) (layer "F.Cu") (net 7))
 (segment (start 198.464365 95.2) (end 201.25 95.2) (width 0.2) (layer "F.Cu") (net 7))
 (segment (start 174.07 81.61) (end 174.07 80.07) (width 0.2) (layer "F.Cu") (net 7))
 (segment (start 174.07 80.07) (end 174 80) (width 0.2) (layer "F.Cu") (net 7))
 (segment (start 201 99) (end 180.5 99) (width 0.2) (layer "F.Cu") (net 7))
 (segment (start 154.2 72.25) (end 151.75 72.25) (width 0.2) (layer "F.Cu") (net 7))
 (segment (start 151.1 84.5) (end 154.5 84.5) (width 0.2) (layer "F.Cu") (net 7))
 (segment (start 178.5 99) (end 157.5 99) (width 0.2) (layer "F.Cu") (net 7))
 (segment (start 171.725 65) (end 169 62.275) (width 0.2) (layer "F.Cu") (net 7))
 (segment (start 176 62.5) (end 176 64.5) (width 0.2) (layer "F.Cu") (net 7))
 (segment (start 153 58.55) (end 153 58.5) (width 0.2) (layer "F.Cu") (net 7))
 (segment (start 182.175635 78) (end 185.33 81.154365) (width 0.2) (layer "F.Cu") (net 7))
 (segment (start 150.6 71.1) (end 150.6 58.5) (width 0.2) (layer "F.Cu") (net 7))
 (segment (start 178.75 98.75) (end 178.5 99) (width 0.2) (layer "F.Cu") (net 7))
 (segment (start 150.6 55) (end 169 55) (width 0.2) (layer "F.Cu") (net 7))
 (segment (start 174 80) (end 174 78) (width 0.2) (layer "F.Cu") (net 7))
 (segment (start 178.75 95.2) (end 178.75 98.75) (width 0.2) (layer "F.Cu") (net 7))
 (segment (start 150.6 58.5) (end 150.6 55) (width 0.2) (layer "F.Cu") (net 7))
 (segment (start 225.4 85.5) (end 225.4 99) (width 0.2) (layer "F.Cu") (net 7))
 (segment (start 225.4 71.5) (end 225.4 85.5) (width 0.2) (layer "F.Cu") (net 7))
 (segment (start 175.5 61.5) (end 175.5 62) (width 0.2) (layer "F.Cu") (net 7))
 (segment (start 150.6 70.5) (end 150.6 84) (width 0.2) (layer "F.Cu") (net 7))
 (segment (start 154.2 59.75) (end 153 58.55) (width 0.2) (layer "F.Cu") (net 7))
 (segment (start 203 99) (end 201 99) (width 0.2) (layer "F.Cu") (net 7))
 (segment (start 180.5 99) (end 178.5 99) (width 0.2) (layer "F.Cu") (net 7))
 (segment (start 157.75 95.2) (end 157.75 98.75) (width 0.2) (layer "F.Cu") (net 7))
 (segment (start 157.5 99) (end 151 99) (width 0.2) (layer "F.Cu") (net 7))
 (segment (start 221.5 85.5) (end 225.4 85.5) (width 0.2) (layer "F.Cu") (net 7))
 (segment (start 150.6 84) (end 151.1 84.5) (width 0.2) (layer "F.Cu") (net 7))
 (segment (start 169 55) (end 175.5 61.5) (width 0.2) (layer "F.Cu") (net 7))
 (segment (start 175.5 65) (end 171.725 65) (width 0.2) (layer "F.Cu") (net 7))
 (segment (start 176 64.5) (end 175.5 65) (width 0.2) (layer "F.Cu") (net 7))
 (segment (start 225.4 99) (end 203 99) (width 0.2) (layer "F.Cu") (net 7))
 (segment (start 174 78) (end 182.175635 78) (width 0.2) (layer "F.Cu") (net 7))
 (segment (start 153 58.5) (end 150.6 58.5) (width 0.2) (layer "F.Cu") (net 7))
 (segment (start 225.4 59.5) (end 225.4 71.5) (width 0.2) (layer "F.Cu") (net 7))
 (segment (start 154.2 74.75) (end 155.95 73) (width 0.2) (layer "F.Cu") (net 15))
 (segment (start 164.5 73) (end 165.5 74) (width 0.2) (layer "F.Cu") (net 15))
 (segment (start 155.95 73) (end 164.5 73) (width 0.2) (layer "F.Cu") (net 15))
 (segment (start 165.5 74) (end 186.78 74) (width 0.2) (layer "F.Cu") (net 15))
 (segment (start 186.78 74) (end 194.39 81.61) (width 0.2) (layer "F.Cu") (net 15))
 (segment (start 202.01 63.49) (end 203.5 62) (width 0.2) (layer "F.Cu") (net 1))
 (segment (start 203.5 62) (end 209.69 62) (width 0.2) (layer "F.Cu") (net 1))
 (segment (start 202.01 66.37) (end 202.01 63.49) (width 0.2) (layer "F.Cu") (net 1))
 (segment (start 217.31 62) (end 221.5 62) (width 0.2) (layer "F.Cu") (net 2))
 (segment (start 217.62 74.5) (end 221 74.5) (width 0.2) (layer "F.Cu") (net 16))
 (segment (start 221 74.5) (end 221.5 74) (width 0.2) (layer "F.Cu") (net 16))
 (segment (start 217.31 88) (end 221.5 88) (width 0.2) (layer "F.Cu") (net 9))
 (segment (start 183.615 62) (end 187.265 58.35) (width 0.2) (layer "F.Cu") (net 4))
 (segment (start 178 58.5) (end 181.5 62) (width 0.2) (layer "F.Cu") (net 4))
 (segment (start 181.5 62) (end 183.615 62) (width 0.2) (layer "F.Cu") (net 4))
 (segment (start 187.915 59) (end 187.547843 58.632843) (width 0.2) (layer "F.Cu") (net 4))
 (segment (start 183.96 55.96) (end 178 55.96) (width 0.2) (layer "F.Cu") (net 3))
 (segment (start 184.725 58.35) (end 184.725 59.895) (width 0.2) (layer "F.Cu") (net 3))
 (segment (start 184.725 56.725) (end 183.96 55.96) (width 0.2) (layer "F.Cu") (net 3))
 (segment (start 184.725 58.35) (end 184.725 56.725) (width 0.2) (layer "F.Cu") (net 3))
 (segment (start 175.5 56) (end 175 55.5) (width 0.2) (layer "F.Cu") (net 5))
 (segment (start 175 55.5) (end 174 55.5) (width 0.2) (layer "F.Cu") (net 5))
 (segment (start 178 61.04) (end 175.5 58.54) (width 0.2) (layer "F.Cu") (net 5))
 (segment (start 175.5 58.54) (end 175.5 56) (width 0.2) (layer "F.Cu") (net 5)))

